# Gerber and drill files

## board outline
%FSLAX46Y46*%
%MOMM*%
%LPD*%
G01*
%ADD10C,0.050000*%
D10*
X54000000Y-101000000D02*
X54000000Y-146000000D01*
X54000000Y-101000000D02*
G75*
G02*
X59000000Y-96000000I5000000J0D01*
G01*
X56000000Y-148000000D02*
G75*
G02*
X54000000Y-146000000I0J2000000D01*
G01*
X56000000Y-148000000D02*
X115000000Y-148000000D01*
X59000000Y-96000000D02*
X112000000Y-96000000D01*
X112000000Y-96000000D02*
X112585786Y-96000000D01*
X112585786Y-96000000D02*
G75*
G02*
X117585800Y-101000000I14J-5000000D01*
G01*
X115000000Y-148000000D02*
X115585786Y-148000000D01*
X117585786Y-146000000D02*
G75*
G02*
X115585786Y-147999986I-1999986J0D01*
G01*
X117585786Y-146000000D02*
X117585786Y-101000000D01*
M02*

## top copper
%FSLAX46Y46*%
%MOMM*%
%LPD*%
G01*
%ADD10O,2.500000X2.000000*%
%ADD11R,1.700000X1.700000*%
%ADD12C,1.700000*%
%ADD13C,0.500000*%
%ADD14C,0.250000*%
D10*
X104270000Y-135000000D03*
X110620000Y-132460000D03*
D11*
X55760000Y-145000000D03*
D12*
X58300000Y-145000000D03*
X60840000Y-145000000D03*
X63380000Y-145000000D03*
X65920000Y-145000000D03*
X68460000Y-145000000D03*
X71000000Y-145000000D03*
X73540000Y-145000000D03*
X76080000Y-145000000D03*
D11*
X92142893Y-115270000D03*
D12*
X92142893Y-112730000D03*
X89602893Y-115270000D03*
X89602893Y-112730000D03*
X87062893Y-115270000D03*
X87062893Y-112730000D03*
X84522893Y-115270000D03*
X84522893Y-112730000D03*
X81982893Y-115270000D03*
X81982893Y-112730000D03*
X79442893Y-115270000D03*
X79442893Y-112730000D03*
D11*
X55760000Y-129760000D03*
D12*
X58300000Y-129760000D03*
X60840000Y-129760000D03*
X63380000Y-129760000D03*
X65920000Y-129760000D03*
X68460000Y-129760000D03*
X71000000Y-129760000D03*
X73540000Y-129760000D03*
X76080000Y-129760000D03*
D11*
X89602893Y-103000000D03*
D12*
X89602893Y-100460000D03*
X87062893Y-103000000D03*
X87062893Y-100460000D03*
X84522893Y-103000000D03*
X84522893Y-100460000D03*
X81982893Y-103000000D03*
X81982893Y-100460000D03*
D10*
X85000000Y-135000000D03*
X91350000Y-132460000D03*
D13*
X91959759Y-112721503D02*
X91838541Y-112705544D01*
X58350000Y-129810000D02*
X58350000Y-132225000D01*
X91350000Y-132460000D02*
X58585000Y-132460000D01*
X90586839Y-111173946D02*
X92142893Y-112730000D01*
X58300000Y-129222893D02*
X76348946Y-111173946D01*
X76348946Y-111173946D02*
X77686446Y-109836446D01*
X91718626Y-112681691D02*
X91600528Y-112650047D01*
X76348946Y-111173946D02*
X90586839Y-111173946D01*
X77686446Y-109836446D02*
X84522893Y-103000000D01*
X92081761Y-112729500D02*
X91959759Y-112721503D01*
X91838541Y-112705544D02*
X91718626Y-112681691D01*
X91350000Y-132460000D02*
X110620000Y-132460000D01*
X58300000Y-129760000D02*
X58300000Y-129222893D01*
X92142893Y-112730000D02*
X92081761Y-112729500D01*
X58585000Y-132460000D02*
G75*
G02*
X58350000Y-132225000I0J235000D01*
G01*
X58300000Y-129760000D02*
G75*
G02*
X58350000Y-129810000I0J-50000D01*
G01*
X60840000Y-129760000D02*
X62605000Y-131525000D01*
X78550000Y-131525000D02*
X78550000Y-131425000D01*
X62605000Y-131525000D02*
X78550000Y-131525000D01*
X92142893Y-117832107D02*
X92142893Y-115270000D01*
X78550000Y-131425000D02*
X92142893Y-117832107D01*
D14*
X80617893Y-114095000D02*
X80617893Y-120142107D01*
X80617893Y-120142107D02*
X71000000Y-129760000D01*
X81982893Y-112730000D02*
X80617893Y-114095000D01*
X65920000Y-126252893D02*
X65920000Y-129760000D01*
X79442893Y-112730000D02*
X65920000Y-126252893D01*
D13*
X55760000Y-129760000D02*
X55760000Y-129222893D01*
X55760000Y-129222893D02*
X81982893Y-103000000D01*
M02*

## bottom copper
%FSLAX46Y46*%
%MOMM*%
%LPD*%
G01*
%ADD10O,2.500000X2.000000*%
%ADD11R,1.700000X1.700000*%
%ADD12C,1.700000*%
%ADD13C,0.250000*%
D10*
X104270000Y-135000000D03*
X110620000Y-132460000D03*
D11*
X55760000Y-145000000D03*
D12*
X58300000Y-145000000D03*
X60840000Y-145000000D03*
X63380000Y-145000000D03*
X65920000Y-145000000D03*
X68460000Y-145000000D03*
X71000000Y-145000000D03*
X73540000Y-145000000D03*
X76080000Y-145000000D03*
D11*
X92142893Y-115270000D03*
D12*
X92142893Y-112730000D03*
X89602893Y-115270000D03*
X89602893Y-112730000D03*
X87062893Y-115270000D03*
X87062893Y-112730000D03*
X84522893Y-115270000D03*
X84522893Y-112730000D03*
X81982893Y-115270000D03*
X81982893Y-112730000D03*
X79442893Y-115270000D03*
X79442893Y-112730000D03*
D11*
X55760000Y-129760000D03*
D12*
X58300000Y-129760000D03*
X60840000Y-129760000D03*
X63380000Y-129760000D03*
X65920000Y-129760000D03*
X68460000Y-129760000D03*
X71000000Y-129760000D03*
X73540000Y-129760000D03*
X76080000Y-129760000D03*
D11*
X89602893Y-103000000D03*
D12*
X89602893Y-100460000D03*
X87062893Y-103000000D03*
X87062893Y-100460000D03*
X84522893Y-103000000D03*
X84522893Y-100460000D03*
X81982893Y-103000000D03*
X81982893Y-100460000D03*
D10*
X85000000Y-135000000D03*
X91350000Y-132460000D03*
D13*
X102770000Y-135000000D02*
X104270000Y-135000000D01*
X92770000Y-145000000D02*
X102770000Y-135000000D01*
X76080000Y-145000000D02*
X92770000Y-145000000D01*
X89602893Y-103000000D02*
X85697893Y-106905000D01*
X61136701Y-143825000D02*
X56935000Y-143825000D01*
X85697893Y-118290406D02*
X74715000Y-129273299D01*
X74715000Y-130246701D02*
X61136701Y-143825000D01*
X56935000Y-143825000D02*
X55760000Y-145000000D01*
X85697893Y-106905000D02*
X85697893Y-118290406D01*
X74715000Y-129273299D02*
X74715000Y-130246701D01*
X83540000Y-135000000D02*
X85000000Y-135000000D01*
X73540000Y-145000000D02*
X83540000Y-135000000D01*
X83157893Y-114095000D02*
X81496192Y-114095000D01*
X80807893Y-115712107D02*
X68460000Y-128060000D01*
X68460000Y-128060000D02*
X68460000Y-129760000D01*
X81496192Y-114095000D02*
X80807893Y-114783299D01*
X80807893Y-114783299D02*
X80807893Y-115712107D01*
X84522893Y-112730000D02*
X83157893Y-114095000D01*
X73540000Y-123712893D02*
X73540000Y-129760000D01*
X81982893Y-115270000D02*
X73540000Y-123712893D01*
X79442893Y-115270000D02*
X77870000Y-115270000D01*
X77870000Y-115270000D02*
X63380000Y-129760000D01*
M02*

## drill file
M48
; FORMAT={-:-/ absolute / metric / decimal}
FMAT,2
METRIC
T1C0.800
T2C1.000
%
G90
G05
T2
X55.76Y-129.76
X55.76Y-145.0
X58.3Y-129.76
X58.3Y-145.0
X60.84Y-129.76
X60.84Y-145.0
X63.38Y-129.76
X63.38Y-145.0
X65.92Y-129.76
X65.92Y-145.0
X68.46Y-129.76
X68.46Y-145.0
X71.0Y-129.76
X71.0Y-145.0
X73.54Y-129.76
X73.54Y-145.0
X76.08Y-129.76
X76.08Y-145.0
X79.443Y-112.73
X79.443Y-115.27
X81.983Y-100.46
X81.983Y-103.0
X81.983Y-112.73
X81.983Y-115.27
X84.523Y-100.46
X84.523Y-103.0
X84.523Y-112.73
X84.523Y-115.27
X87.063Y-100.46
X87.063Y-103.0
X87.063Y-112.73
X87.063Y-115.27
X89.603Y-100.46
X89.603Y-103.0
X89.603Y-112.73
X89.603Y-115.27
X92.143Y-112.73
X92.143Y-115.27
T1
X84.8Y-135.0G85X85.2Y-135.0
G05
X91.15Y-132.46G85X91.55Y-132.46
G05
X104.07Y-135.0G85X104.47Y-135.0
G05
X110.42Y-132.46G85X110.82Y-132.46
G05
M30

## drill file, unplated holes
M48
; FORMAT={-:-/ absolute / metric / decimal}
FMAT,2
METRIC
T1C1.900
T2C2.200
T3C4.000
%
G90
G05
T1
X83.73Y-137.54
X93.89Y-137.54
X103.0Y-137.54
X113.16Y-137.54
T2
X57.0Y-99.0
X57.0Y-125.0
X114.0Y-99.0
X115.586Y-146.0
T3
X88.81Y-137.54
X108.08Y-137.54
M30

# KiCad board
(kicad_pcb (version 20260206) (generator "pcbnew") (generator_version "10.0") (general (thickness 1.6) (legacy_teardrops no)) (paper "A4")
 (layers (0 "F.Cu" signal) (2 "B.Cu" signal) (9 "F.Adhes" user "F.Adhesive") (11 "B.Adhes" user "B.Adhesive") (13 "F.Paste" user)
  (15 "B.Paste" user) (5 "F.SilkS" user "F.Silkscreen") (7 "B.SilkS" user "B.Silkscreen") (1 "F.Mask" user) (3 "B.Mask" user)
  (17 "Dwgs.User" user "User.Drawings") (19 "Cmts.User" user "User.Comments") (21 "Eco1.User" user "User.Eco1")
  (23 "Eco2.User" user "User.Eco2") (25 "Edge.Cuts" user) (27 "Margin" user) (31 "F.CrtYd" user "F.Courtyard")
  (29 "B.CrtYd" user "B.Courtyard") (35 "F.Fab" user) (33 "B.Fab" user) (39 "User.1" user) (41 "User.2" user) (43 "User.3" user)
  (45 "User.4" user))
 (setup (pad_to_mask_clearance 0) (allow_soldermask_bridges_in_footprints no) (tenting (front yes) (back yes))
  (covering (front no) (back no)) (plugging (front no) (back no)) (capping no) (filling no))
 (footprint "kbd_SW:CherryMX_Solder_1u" (layer "F.Cu") (at 108.08 137.54)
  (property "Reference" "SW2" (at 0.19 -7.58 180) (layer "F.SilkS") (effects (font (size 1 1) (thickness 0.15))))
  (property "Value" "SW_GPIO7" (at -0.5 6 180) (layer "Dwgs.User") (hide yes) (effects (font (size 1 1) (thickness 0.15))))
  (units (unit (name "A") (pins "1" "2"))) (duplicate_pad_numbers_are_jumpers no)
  (pad "" np_thru_hole circle (at -5.08 0 90) (size 1.9 1.9) (drill 1.9) (layers "*.Cu" "*.Mask"))
  (pad "" np_thru_hole circle (at 0 0 90) (size 4 4) (drill 4) (layers "*.Cu" "*.Mask"))
  (pad "" np_thru_hole circle (at 5.08 0 90) (size 1.9 1.9) (drill 1.9) (layers "*.Cu" "*.Mask"))
  (pad "1" thru_hole oval (at -3.81 -2.54) (size 2.5 2) (drill oval 1.2 0.8) (layers "*.Cu" "B.Mask" "F.SilkS") (remove_unused_layers no)
   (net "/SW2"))
  (pad "2" thru_hole oval (at 2.54 -5.08) (size 2.5 2) (drill oval 1.2 0.8) (layers "*.Cu" "B.Mask" "F.SilkS") (remove_unused_layers no)
   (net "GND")))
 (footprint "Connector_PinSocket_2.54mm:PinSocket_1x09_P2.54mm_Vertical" (layer "F.Cu") (at 55.76 145 90)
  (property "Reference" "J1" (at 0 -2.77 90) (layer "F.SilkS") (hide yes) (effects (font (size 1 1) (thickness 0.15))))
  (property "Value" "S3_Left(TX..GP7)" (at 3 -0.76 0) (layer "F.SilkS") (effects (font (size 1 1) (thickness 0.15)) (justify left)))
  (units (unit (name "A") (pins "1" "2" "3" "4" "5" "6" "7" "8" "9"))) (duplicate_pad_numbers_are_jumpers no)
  (pad "1" thru_hole rect (at 0 0 90) (size 1.7 1.7) (drill 1) (layers "*.Cu" "*.Mask") (remove_unused_layers no) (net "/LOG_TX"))
  (pad "2" thru_hole circle (at 0 2.54 90) (size 1.7 1.7) (drill 1) (layers "*.Cu" "*.Mask") (remove_unused_layers no)
   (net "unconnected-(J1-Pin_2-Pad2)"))
  (pad "3" thru_hole circle (at 0 5.08 90) (size 1.7 1.7) (drill 1) (layers "*.Cu" "*.Mask") (remove_unused_layers no)
   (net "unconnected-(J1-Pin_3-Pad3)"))
  (pad "4" thru_hole circle (at 0 7.62 90) (size 1.7 1.7) (drill 1) (layers "*.Cu" "*.Mask") (remove_unused_layers no)
   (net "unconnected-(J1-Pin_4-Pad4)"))
  (pad "5" thru_hole circle (at 0 10.16 90) (size 1.7 1.7) (drill 1) (layers "*.Cu" "*.Mask") (remove_unused_layers no)
   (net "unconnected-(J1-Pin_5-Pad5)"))
  (pad "6" thru_hole circle (at 0 12.7 90) (size 1.7 1.7) (drill 1) (layers "*.Cu" "*.Mask") (remove_unused_layers no)
   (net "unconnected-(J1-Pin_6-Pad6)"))
  (pad "7" thru_hole circle (at 0 15.24 90) (size 1.7 1.7) (drill 1) (layers "*.Cu" "*.Mask") (remove_unused_layers no)
   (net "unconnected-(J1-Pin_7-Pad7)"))
  (pad "8" thru_hole circle (at 0 17.78 90) (size 1.7 1.7) (drill 1) (layers "*.Cu" "*.Mask") (remove_unused_layers no) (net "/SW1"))
  (pad "9" thru_hole circle (at 0 20.32 90) (size 1.7 1.7) (drill 1) (layers "*.Cu" "*.Mask") (remove_unused_layers no) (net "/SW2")))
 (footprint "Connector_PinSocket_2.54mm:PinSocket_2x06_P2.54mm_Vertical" (layer "F.Cu") (at 92.142893 115.27 -90)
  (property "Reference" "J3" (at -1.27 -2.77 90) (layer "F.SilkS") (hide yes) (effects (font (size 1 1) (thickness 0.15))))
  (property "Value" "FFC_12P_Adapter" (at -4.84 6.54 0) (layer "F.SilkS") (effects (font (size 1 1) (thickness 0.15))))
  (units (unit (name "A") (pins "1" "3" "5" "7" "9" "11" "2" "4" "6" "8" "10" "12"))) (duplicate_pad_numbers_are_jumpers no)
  (pad "1" thru_hole rect (at 0 0 270) (size 1.7 1.7) (drill 1) (layers "*.Cu" "*.Mask") (remove_unused_layers no) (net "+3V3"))
  (pad "2" thru_hole circle (at -2.54 0 270) (size 1.7 1.7) (drill 1) (layers "*.Cu" "*.Mask") (remove_unused_layers no) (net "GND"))
  (pad "3" thru_hole circle (at 0 2.54 270) (size 1.7 1.7) (drill 1) (layers "*.Cu" "*.Mask") (remove_unused_layers no)
   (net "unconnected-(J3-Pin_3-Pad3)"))
  (pad "4" thru_hole circle (at -2.54 2.54 270) (size 1.7 1.7) (drill 1) (layers "*.Cu" "*.Mask") (remove_unused_layers no)
   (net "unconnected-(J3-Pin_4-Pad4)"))
  (pad "5" thru_hole circle (at 0 5.08 270) (size 1.7 1.7) (drill 1) (layers "*.Cu" "*.Mask") (remove_unused_layers no)
   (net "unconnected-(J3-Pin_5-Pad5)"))
  (pad "6" thru_hole circle (at -2.54 5.08 270) (size 1.7 1.7) (drill 1) (layers "*.Cu" "*.Mask") (remove_unused_layers no)
   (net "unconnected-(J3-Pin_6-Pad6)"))
  (pad "7" thru_hole circle (at 0 7.62 270) (size 1.7 1.7) (drill 1) (layers "*.Cu" "*.Mask") (remove_unused_layers no)
   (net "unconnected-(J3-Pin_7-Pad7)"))
  (pad "8" thru_hole circle (at -2.54 7.62 270) (size 1.7 1.7) (drill 1) (layers "*.Cu" "*.Mask") (remove_unused_layers no) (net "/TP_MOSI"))
  (pad "9" thru_hole circle (at 0 10.16 270) (size 1.7 1.7) (drill 1) (layers "*.Cu" "*.Mask") (remove_unused_layers no) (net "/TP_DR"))
  (pad "10" thru_hole circle (at -2.54 10.16 270) (size 1.7 1.7) (drill 1) (layers "*.Cu" "*.Mask") (remove_unused_layers no) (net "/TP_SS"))
  (pad "11" thru_hole circle (at 0 12.7 270) (size 1.7 1.7) (drill 1) (layers "*.Cu" "*.Mask") (remove_unused_layers no) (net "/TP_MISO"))
  (pad "12" thru_hole circle (at -2.54 12.7 270) (size 1.7 1.7) (drill 1) (layers "*.Cu" "*.Mask") (remove_unused_layers no) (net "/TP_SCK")))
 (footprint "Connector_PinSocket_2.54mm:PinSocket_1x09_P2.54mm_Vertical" (layer "F.Cu") (at 55.76 129.76 90)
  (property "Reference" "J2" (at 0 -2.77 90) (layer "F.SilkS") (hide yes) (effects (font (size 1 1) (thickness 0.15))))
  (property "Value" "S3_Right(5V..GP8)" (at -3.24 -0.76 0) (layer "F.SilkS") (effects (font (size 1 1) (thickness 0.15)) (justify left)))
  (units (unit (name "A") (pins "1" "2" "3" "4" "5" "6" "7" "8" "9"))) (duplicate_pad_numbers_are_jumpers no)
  (pad "1" thru_hole rect (at 0 0 90) (size 1.7 1.7) (drill 1) (layers "*.Cu" "*.Mask") (remove_unused_layers no) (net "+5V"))
  (pad "2" thru_hole circle (at 0 2.54 90) (size 1.7 1.7) (drill 1) (layers "*.Cu" "*.Mask") (remove_unused_layers no) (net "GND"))
  (pad "3" thru_hole circle (at 0 5.08 90) (size 1.7 1.7) (drill 1) (layers "*.Cu" "*.Mask") (remove_unused_layers no) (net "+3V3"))
  (pad "4" thru_hole circle (at 0 7.62 90) (size 1.7 1.7) (drill 1) (layers "*.Cu" "*.Mask") (remove_unused_layers no) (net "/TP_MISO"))
  (pad "5" thru_hole circle (at 0 10.16 90) (size 1.7 1.7) (drill 1) (layers "*.Cu" "*.Mask") (remove_unused_layers no) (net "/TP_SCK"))
  (pad "6" thru_hole circle (at 0 12.7 90) (size 1.7 1.7) (drill 1) (layers "*.Cu" "*.Mask") (remove_unused_layers no) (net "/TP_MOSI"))
  (pad "7" thru_hole circle (at 0 15.24 90) (size 1.7 1.7) (drill 1) (layers "*.Cu" "*.Mask") (remove_unused_layers no) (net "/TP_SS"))
  (pad "8" thru_hole circle (at 0 17.78 90) (size 1.7 1.7) (drill 1) (layers "*.Cu" "*.Mask") (remove_unused_layers no) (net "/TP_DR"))
  (pad "9" thru_hole circle (at 0 20.32 90) (size 1.7 1.7) (drill 1) (layers "*.Cu" "*.Mask") (remove_unused_layers no)
   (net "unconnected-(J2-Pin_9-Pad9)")))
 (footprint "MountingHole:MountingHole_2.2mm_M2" (layer "F.Cu") (at 57 125)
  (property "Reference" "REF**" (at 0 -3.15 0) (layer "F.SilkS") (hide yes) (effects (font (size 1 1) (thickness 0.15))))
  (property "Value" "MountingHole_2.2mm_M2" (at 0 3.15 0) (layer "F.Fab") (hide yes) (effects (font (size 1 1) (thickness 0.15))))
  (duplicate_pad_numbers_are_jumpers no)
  (pad "" np_thru_hole circle (at 0 0) (size 2.2 2.2) (drill 2.2) (layers "*.Cu" "*.Mask")))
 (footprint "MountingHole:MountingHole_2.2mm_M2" (layer "F.Cu") (at 57 99)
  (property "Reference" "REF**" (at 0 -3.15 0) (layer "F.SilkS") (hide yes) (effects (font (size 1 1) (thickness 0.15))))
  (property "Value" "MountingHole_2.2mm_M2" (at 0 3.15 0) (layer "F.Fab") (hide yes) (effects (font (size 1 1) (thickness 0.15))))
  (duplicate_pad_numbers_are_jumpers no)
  (pad "" np_thru_hole circle (at 0 0) (size 2.2 2.2) (drill 2.2) (layers "*.Cu" "*.Mask")))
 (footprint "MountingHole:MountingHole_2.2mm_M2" (layer "F.Cu") (at 114 99)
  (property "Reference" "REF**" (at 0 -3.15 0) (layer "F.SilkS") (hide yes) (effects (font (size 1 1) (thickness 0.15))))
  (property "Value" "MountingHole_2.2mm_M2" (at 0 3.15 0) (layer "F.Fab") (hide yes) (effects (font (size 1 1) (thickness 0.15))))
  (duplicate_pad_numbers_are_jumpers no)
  (pad "" np_thru_hole circle (at 0 0) (size 2.2 2.2) (drill 2.2) (layers "*.Cu" "*.Mask")))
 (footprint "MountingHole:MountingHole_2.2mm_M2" (layer "F.Cu") (at 115.5858 146)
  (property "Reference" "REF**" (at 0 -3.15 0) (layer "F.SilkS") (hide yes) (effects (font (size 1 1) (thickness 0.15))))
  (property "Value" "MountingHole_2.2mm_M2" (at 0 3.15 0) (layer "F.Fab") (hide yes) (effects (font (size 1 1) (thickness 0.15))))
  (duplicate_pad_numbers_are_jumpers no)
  (pad "" np_thru_hole circle (at 0 0) (size 2.2 2.2) (drill 2.2) (layers "*.Cu" "*.Mask")))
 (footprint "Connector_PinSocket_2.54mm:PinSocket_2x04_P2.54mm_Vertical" (layer "F.Cu") (at 89.602893 103 -90)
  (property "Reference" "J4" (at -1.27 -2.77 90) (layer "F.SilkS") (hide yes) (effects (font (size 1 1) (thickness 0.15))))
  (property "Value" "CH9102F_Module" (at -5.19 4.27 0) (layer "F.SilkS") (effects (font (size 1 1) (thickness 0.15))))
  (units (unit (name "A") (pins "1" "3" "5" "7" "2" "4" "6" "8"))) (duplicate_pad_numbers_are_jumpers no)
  (pad "1" thru_hole rect (at 0 0 270) (size 1.7 1.7) (drill 1) (layers "*.Cu" "*.Mask") (remove_unused_layers no) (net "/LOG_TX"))
  (pad "2" thru_hole circle (at -2.54 0 270) (size 1.7 1.7) (drill 1) (layers "*.Cu" "*.Mask") (remove_unused_layers no)
   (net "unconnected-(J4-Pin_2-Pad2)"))
  (pad "3" thru_hole circle (at 0 2.54 270) (size 1.7 1.7) (drill 1) (layers "*.Cu" "*.Mask") (remove_unused_layers no)
   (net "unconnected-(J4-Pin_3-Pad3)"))
  (pad "4" thru_hole circle (at -2.54 2.54 270) (size 1.7 1.7) (drill 1) (layers "*.Cu" "*.Mask") (remove_unused_layers no)
   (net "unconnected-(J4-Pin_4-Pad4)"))
  (pad "5" thru_hole circle (at 0 5.08 270) (size 1.7 1.7) (drill 1) (layers "*.Cu" "*.Mask") (remove_unused_layers no) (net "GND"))
  (pad "6" thru_hole circle (at -2.54 5.08 270) (size 1.7 1.7) (drill 1) (layers "*.Cu" "*.Mask") (remove_unused_layers no)
   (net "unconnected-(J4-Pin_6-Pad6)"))
  (pad "7" thru_hole circle (at 0 7.62 270) (size 1.7 1.7) (drill 1) (layers "*.Cu" "*.Mask") (remove_unused_layers no) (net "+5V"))
  (pad "8" thru_hole circle (at -2.54 7.62 270) (size 1.7 1.7) (drill 1) (layers "*.Cu" "*.Mask") (remove_unused_layers no)
   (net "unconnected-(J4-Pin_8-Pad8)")))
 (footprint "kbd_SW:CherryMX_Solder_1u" (layer "F.Cu") (at 88.81 137.54)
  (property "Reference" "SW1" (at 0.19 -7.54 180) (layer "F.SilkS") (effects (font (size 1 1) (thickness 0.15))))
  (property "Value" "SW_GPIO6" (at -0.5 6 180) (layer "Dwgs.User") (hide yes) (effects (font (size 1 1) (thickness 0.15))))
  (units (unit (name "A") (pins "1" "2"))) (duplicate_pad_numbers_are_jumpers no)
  (pad "" np_thru_hole circle (at -5.08 0 90) (size 1.9 1.9) (drill 1.9) (layers "*.Cu" "*.Mask"))
  (pad "" np_thru_hole circle (at 0 0 90) (size 4 4) (drill 4) (layers "*.Cu" "*.Mask"))
  (pad "" np_thru_hole circle (at 5.08 0 90) (size 1.9 1.9) (drill 1.9) (layers "*.Cu" "*.Mask"))
  (pad "1" thru_hole oval (at -3.81 -2.54) (size 2.5 2) (drill oval 1.2 0.8) (layers "*.Cu" "B.Mask" "F.SilkS") (remove_unused_layers no)
   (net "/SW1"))
  (pad "2" thru_hole oval (at 2.54 -5.08) (size 2.5 2) (drill oval 1.2 0.8) (layers "*.Cu" "B.Mask" "F.SilkS") (remove_unused_layers no)
   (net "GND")))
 (gr_line (start 54 101) (end 54 146) (stroke (width 0.05) (type solid)) (layer "Edge.Cuts"))
 (gr_arc (start 54 101) (mid 55.464466 97.464466) (end 59 96) (stroke (width 0.05) (type default)) (layer "Edge.Cuts"))
 (gr_arc (start 56 148) (mid 54.585786 147.414214) (end 54 146) (stroke (width 0.05) (type default)) (layer "Edge.Cuts"))
 (gr_line (start 56 148) (end 115 148) (stroke (width 0.05) (type default)) (layer "Edge.Cuts"))
 (gr_line (start 59 96) (end 112 96) (stroke (width 0.05) (type default)) (layer "Edge.Cuts"))
 (gr_line (start 112 96) (end 112.585786 96) (stroke (width 0.05) (type default)) (layer "Edge.Cuts"))
 (gr_arc (start 112.585786 96) (mid 116.12132 97.464466) (end 117.585786 101) (stroke (width 0.05) (type default)) (layer "Edge.Cuts"))
 (gr_line (start 115 148) (end 115.585786 148) (stroke (width 0.05) (type default)) (layer "Edge.Cuts"))
 (gr_arc (start 117.585786 146) (mid 116.999999 147.414209) (end 115.585786 148) (stroke (width 0.05) (type default)) (layer "Edge.Cuts"))
 (gr_line (start 117.585786 146) (end 117.585786 101) (stroke (width 0.05) (type default)) (layer "Edge.Cuts"))
 (segment (start 102.77 135) (end 104.27 135) (width 0.25) (layer "B.Cu") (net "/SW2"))
 (segment (start 92.77 145) (end 102.77 135) (width 0.25) (layer "B.Cu") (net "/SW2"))
 (segment (start 76.08 145) (end 92.77 145) (width 0.25) (layer "B.Cu") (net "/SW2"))
 (segment (start 91.959759 112.721503) (end 91.838541 112.705544) (width 0.5) (layer "F.Cu") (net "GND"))
 (segment (start 58.35 129.81) (end 58.35 132.225) (width 0.5) (layer "F.Cu") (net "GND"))
 (segment (start 91.35 132.46) (end 58.585 132.46) (width 0.5) (layer "F.Cu") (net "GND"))
 (segment (start 90.586839 111.173946) (end 92.142893 112.73) (width 0.5) (layer "F.Cu") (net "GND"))
 (segment (start 58.3 129.222893) (end 76.348946 111.173946) (width 0.5) (layer "F.Cu") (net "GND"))
 (segment (start 76.348946 111.173946) (end 77.686446 109.836446) (width 0.5) (layer "F.Cu") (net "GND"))
 (segment (start 91.718626 112.681691) (end 91.600528 112.650047) (width 0.5) (layer "F.Cu") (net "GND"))
 (segment (start 76.348946 111.173946) (end 90.586839 111.173946) (width 0.5) (layer "F.Cu") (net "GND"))
 (segment (start 77.686446 109.836446) (end 84.522893 103) (width 0.5) (layer "F.Cu") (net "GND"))
 (segment (start 92.081761 112.7295) (end 91.959759 112.721503) (width 0.5) (layer "F.Cu") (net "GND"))
 (segment (start 91.838541 112.705544) (end 91.718626 112.681691) (width 0.5) (layer "F.Cu") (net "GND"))
 (segment (start 91.35 132.46) (end 110.62 132.46) (width 0.5) (layer "F.Cu") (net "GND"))
 (segment (start 58.3 129.76) (end 58.3 129.222893) (width 0.5) (layer "F.Cu") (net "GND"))
 (segment (start 92.142893 112.73) (end 92.081761 112.7295) (width 0.5) (layer "F.Cu") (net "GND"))
 (arc (start 58.585 132.46) (mid 58.41883 132.39117) (end 58.35 132.225) (width 0.5) (layer "F.Cu") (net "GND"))
 (arc (start 58.3 129.76) (mid 58.335355 129.774645) (end 58.35 129.81) (width 0.5) (layer "F.Cu") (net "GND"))
 (segment (start 89.602893 103) (end 85.697893 106.905) (width 0.25) (layer "B.Cu") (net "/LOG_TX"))
 (segment (start 61.136701 143.825) (end 56.935 143.825) (width 0.25) (layer "B.Cu") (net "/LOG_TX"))
 (segment (start 85.697893 118.290406) (end 74.715 129.273299) (width 0.25) (layer "B.Cu") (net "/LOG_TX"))
 (segment (start 74.715 130.246701) (end 61.136701 143.825) (width 0.25) (layer "B.Cu") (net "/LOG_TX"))
 (segment (start 56.935 143.825) (end 55.76 145) (width 0.25) (layer "B.Cu") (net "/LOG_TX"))
 (segment (start 85.697893 106.905) (end 85.697893 118.290406) (width 0.25) (layer "B.Cu") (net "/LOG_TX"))
 (segment (start 74.715 129.273299) (end 74.715 130.246701) (width 0.25) (layer "B.Cu") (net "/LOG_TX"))
 (segment (start 83.54 135) (end 85 135) (width 0.25) (layer "B.Cu") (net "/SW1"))
 (segment (start 73.54 145) (end 83.54 135) (width 0.25) (layer "B.Cu") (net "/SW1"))
 (segment (start 60.84 129.76) (end 62.605 131.525) (width 0.5) (layer "F.Cu") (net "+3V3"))
 (segment (start 78.55 131.525) (end 78.55 131.425) (width 0.5) (layer "F.Cu") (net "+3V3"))
 (segment (start 62.605 131.525) (end 78.55 131.525) (width 0.5) (layer "F.Cu") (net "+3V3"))
 (segment (start 92.142893 117.832107) (end 92.142893 115.27) (width 0.5) (layer "F.Cu") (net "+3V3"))
 (segment (start 78.55 131.425) (end 92.142893 117.832107) (width 0.5) (layer "F.Cu") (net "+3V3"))
 (segment (start 83.157893 114.095) (end 81.496192 114.095) (width 0.25) (layer "B.Cu") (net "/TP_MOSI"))
 (segment (start 80.807893 115.712107) (end 68.46 128.06) (width 0.25) (layer "B.Cu") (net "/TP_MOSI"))
 (segment (start 68.46 128.06) (end 68.46 129.76) (width 0.25) (layer "B.Cu") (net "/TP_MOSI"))
 (segment (start 81.496192 114.095) (end 80.807893 114.783299) (width 0.25) (layer "B.Cu") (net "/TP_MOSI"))
 (segment (start 80.807893 114.783299) (end 80.807893 115.712107) (width 0.25) (layer "B.Cu") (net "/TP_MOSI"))
 (segment (start 84.522893 112.73) (end 83.157893 114.095) (width 0.25) (layer "B.Cu") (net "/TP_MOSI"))
 (segment (start 73.54 123.712893) (end 73.54 129.76) (width 0.25) (layer "B.Cu") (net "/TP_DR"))
 (segment (start 81.982893 115.27) (end 73.54 123.712893) (width 0.25) (layer "B.Cu") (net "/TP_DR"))
 (segment (start 80.617893 114.095) (end 80.617893 120.142107) (width 0.25) (layer "F.Cu") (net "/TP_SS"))
 (segment (start 80.617893 120.142107) (end 71 129.76) (width 0.25) (layer "F.Cu") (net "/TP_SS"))
 (segment (start 81.982893 112.73) (end 80.617893 114.095) (width 0.25) (layer "F.Cu") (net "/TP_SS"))
 (segment (start 79.442893 115.27) (end 77.87 115.27) (width 0.25) (layer "B.Cu") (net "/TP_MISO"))
 (segment (start 77.87 115.27) (end 63.38 129.76) (width 0.25) (layer "B.Cu") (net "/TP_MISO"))
 (segment (start 65.92 126.252893) (end 65.92 129.76) (width 0.25) (layer "F.Cu") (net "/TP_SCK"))
 (segment (start 79.442893 112.73) (end 65.92 126.252893) (width 0.25) (layer "F.Cu") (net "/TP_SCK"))
 (segment (start 55.76 129.76) (end 55.76 129.222893) (width 0.5) (layer "F.Cu") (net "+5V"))
 (segment (start 55.76 129.222893) (end 81.982893 103) (width 0.5) (layer "F.Cu") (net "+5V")))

